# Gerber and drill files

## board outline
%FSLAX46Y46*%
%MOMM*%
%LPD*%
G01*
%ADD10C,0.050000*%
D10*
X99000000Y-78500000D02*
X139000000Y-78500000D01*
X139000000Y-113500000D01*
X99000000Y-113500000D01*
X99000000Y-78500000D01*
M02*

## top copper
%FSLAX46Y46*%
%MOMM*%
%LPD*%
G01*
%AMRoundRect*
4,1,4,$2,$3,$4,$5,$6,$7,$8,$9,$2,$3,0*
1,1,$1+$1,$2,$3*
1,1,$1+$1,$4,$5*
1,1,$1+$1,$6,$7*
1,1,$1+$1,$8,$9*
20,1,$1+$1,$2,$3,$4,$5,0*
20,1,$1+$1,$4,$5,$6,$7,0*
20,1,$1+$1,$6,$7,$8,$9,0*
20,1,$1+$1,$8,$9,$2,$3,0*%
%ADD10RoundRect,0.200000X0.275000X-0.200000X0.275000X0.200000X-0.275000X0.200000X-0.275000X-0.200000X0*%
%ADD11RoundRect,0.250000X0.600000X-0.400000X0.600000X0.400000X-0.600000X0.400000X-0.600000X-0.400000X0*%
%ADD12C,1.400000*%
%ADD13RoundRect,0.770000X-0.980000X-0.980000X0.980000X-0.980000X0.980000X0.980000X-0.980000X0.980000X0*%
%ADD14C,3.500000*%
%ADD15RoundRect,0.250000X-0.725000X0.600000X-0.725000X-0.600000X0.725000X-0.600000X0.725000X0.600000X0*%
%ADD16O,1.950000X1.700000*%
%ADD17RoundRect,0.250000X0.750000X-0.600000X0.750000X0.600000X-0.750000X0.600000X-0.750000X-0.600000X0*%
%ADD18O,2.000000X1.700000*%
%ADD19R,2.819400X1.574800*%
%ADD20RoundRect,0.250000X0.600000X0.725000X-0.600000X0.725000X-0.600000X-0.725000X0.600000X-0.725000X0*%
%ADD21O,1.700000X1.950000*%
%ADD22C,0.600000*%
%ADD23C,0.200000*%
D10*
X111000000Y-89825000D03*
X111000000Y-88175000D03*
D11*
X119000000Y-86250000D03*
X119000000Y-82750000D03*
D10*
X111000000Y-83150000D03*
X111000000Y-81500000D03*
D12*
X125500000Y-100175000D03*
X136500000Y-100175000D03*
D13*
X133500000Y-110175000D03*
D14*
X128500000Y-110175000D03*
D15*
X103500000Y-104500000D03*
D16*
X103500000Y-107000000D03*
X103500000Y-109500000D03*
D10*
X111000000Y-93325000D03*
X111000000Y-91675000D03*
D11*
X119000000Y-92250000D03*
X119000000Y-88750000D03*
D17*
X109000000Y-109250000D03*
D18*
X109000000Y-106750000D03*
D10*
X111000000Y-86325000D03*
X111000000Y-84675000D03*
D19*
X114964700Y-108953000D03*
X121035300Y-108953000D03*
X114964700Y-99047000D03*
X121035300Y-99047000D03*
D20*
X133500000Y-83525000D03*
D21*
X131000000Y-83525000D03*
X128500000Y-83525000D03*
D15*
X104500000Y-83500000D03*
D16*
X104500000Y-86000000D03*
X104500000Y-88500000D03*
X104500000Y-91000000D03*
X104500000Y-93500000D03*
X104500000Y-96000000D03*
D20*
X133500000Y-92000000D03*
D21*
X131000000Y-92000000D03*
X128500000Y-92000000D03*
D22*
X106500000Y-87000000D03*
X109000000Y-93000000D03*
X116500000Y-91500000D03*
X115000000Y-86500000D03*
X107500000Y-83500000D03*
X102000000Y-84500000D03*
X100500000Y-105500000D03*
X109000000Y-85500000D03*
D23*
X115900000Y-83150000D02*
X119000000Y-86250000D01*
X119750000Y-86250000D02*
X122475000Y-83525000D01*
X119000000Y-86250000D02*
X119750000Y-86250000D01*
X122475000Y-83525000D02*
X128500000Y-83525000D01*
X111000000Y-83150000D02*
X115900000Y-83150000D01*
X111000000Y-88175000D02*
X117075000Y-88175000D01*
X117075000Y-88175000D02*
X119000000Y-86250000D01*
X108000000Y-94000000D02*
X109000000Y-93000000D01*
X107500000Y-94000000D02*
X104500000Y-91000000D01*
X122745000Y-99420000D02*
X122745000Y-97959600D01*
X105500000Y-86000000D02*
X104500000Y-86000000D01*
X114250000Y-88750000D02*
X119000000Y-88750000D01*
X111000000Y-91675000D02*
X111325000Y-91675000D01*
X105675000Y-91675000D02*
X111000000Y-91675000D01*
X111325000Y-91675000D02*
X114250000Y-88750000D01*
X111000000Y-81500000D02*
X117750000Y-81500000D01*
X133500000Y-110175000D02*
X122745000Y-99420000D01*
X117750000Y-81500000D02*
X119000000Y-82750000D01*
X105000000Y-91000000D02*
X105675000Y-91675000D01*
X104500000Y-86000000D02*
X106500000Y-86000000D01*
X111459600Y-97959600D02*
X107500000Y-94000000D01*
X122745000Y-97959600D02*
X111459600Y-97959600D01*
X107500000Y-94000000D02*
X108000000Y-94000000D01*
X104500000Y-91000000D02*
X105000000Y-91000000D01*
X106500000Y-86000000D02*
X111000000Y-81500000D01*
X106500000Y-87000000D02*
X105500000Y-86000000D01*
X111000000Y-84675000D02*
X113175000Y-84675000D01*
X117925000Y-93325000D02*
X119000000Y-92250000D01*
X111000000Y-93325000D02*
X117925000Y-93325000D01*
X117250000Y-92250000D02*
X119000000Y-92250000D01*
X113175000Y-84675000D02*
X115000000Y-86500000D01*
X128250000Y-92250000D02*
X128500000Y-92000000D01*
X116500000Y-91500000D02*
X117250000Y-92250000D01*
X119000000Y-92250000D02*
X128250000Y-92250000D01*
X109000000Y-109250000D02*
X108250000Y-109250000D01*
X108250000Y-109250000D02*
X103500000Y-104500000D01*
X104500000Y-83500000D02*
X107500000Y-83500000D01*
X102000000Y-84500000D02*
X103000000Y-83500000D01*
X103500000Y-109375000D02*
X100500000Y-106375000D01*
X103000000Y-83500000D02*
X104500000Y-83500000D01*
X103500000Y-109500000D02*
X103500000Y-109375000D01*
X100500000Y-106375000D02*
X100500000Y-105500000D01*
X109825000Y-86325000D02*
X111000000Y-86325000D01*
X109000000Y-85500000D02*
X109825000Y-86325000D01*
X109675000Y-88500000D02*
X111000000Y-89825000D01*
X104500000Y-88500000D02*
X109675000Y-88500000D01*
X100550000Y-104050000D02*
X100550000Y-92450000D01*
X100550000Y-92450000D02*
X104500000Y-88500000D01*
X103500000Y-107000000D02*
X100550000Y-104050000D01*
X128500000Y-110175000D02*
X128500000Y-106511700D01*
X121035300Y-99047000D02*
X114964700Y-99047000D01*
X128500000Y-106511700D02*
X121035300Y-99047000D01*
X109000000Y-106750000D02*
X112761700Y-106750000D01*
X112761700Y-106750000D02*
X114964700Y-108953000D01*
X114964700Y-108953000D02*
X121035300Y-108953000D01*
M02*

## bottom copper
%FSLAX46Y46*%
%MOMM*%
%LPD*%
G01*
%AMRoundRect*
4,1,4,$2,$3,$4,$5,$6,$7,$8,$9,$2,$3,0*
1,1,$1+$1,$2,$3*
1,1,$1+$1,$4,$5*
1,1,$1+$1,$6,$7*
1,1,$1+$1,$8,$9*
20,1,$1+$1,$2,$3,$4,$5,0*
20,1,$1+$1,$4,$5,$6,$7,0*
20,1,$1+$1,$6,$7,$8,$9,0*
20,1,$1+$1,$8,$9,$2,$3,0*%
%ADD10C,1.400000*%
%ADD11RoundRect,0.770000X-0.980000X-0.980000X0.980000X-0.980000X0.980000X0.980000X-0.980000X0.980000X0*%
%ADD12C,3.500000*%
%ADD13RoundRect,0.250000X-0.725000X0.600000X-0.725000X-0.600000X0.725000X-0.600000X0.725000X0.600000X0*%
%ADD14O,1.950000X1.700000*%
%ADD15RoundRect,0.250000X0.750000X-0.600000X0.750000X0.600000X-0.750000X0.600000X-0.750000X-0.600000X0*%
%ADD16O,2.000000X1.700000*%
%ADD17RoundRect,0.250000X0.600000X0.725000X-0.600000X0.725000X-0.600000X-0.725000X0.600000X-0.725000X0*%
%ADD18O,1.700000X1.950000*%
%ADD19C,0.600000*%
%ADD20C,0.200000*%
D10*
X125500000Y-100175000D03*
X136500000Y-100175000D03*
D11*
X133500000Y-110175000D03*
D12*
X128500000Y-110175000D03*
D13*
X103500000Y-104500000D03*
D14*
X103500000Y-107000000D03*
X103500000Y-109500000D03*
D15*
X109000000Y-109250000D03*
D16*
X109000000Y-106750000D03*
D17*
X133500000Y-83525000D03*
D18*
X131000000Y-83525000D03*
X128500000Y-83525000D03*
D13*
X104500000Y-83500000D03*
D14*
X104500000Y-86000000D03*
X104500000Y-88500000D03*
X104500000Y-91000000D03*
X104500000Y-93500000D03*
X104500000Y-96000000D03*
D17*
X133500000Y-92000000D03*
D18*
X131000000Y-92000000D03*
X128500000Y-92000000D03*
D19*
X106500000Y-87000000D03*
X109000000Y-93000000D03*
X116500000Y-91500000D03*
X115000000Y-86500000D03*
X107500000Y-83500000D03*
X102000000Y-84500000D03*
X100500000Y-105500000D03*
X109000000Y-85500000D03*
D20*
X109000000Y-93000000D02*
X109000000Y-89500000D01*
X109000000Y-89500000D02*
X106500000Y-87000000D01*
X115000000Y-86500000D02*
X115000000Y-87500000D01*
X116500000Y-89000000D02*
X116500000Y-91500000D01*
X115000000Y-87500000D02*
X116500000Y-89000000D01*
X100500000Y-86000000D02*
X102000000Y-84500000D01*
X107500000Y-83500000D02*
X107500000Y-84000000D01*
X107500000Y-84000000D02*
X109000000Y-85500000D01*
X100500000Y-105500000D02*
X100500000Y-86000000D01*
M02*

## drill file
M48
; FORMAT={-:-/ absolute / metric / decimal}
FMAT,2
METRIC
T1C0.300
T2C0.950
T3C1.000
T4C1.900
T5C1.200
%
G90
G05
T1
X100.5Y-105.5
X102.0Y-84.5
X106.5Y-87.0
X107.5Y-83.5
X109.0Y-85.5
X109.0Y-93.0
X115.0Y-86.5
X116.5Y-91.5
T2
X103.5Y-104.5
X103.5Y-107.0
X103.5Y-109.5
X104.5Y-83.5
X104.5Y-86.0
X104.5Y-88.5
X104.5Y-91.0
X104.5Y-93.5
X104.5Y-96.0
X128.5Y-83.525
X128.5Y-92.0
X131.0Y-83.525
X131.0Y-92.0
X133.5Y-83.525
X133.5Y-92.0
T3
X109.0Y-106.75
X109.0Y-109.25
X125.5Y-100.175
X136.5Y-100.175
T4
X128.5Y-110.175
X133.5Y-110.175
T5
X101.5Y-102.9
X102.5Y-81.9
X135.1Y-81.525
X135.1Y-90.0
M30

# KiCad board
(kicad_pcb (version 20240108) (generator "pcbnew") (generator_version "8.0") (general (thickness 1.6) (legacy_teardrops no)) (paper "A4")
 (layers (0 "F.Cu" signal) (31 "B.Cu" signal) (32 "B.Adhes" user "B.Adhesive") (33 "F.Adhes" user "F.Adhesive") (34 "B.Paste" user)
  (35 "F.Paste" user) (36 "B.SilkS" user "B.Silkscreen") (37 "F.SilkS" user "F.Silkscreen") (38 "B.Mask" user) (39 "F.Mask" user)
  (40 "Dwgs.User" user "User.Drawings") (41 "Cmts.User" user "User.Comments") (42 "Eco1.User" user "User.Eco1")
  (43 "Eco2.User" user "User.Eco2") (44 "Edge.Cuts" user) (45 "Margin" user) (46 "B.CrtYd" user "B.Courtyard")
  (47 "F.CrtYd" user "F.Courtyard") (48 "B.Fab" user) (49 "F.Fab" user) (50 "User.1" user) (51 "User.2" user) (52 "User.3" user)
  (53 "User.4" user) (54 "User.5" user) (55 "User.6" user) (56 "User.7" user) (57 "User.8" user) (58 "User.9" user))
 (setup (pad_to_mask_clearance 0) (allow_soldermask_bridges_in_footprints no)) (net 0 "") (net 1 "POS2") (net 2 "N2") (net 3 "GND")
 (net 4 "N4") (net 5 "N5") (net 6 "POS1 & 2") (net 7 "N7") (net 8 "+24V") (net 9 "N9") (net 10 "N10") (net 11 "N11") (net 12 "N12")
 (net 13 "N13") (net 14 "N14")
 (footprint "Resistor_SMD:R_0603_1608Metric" (layer "F.Cu") (at 111 89 90)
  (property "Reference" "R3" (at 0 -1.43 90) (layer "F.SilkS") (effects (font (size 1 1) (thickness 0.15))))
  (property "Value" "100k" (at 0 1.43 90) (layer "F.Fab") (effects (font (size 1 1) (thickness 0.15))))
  (pad "1" smd roundrect (at -0.825 0 90) (size 0.8 0.95) (layers "F.Cu" "F.Paste" "F.Mask") (roundrect_rratio 0.25) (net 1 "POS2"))
  (pad "2" smd roundrect (at 0.825 0 90) (size 0.8 0.95) (layers "F.Cu" "F.Paste" "F.Mask") (roundrect_rratio 0.25) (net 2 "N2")))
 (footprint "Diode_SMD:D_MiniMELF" (layer "F.Cu") (at 119 84.5 90)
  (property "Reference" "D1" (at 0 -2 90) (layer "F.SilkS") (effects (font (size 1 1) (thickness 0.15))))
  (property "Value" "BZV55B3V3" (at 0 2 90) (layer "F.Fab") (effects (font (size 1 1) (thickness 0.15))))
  (pad "1" smd roundrect (at -1.75 0 90) (size 1.3 1.7) (layers "F.Cu" "F.Paste" "F.Mask") (roundrect_rratio 0.1923076923) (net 2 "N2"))
  (pad "2" smd roundrect (at 1.75 0 90) (size 1.3 1.7) (layers "F.Cu" "F.Paste" "F.Mask") (roundrect_rratio 0.1923076923) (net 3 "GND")))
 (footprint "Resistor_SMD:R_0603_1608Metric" (layer "F.Cu") (at 111 82.325 90)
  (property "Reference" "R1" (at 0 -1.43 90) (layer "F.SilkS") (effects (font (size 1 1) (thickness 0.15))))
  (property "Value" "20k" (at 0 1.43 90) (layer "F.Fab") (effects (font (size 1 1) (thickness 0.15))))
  (pad "1" smd roundrect (at -0.825 0 90) (size 0.8 0.95) (layers "F.Cu" "F.Paste" "F.Mask") (roundrect_rratio 0.25) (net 2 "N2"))
  (pad "2" smd roundrect (at 0.825 0 90) (size 0.8 0.95) (layers "F.Cu" "F.Paste" "F.Mask") (roundrect_rratio 0.25) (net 3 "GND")))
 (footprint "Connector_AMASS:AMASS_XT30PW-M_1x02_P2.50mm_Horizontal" (layer "F.Cu") (at 133.5 110.175)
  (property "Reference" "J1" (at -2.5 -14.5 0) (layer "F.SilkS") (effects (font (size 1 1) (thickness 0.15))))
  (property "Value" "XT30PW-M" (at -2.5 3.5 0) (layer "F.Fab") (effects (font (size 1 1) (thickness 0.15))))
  (pad "" thru_hole circle (at -8 -10) (size 1.4 1.4) (drill 1) (layers "*.Cu" "*.Mask") (remove_unused_layers no))
  (pad "" thru_hole circle (at 3 -10) (size 1.4 1.4) (drill 1) (layers "*.Cu" "*.Mask") (remove_unused_layers no))
  (pad "1" thru_hole roundrect (at 0 0) (size 3.5 3.5) (drill 1.9) (layers "*.Cu" "*.Mask") (remove_unused_layers no)
   (roundrect_rratio 0.22) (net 3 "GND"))
  (pad "2" thru_hole circle (at -5 0) (size 3.5 3.5) (drill 1.9) (layers "*.Cu" "*.Mask") (remove_unused_layers no) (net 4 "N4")))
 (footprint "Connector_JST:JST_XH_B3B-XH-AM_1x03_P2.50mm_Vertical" (layer "F.Cu") (at 103.5 104.5 -90)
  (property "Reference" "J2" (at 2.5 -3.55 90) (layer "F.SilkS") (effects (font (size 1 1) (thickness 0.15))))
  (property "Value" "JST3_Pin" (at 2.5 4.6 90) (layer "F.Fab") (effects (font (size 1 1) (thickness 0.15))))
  (pad "" np_thru_hole circle (at -1.6 2 270) (size 1.2 1.2) (drill 1.2) (layers "*.Cu" "*.Mask"))
  (pad "1" thru_hole roundrect (at 0 0 270) (size 1.7 1.95) (drill 0.95) (layers "*.Cu" "*.Mask") (remove_unused_layers no)
   (roundrect_rratio 0.147059) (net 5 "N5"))
  (pad "2" thru_hole oval (at 2.5 0 270) (size 1.7 1.95) (drill 0.95) (layers "*.Cu" "*.Mask") (remove_unused_layers no) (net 1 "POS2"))
  (pad "3" thru_hole oval (at 5 0 270) (size 1.7 1.95) (drill 0.95) (layers "*.Cu" "*.Mask") (remove_unused_layers no) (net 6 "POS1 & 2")))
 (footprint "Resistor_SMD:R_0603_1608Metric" (layer "F.Cu") (at 111 92.5 90)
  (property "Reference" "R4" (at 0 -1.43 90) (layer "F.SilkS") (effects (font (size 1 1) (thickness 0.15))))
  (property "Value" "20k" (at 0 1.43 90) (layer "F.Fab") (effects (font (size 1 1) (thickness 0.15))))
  (pad "1" smd roundrect (at -0.825 0 90) (size 0.8 0.95) (layers "F.Cu" "F.Paste" "F.Mask") (roundrect_rratio 0.25) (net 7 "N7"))
  (pad "2" smd roundrect (at 0.825 0 90) (size 0.8 0.95) (layers "F.Cu" "F.Paste" "F.Mask") (roundrect_rratio 0.25) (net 3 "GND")))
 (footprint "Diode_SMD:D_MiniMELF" (layer "F.Cu") (at 119 90.5 90)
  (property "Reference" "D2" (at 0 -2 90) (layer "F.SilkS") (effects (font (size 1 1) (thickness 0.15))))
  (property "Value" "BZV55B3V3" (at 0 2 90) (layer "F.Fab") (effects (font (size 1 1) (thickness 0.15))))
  (pad "1" smd roundrect (at -1.75 0 90) (size 1.3 1.7) (layers "F.Cu" "F.Paste" "F.Mask") (roundrect_rratio 0.1923076923) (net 7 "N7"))
  (pad "2" smd roundrect (at 1.75 0 90) (size 1.3 1.7) (layers "F.Cu" "F.Paste" "F.Mask") (roundrect_rratio 0.1923076923) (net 3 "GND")))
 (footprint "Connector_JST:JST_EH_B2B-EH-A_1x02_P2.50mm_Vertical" (layer "F.Cu") (at 109 109.25 90)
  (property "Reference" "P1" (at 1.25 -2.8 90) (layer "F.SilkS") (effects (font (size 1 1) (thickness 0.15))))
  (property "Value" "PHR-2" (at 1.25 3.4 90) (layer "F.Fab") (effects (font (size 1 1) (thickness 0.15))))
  (pad "1" thru_hole roundrect (at 0 0 90) (size 1.7 2) (drill 1) (layers "*.Cu" "*.Mask") (remove_unused_layers no)
   (roundrect_rratio 0.147059) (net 5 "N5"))
  (pad "2" thru_hole oval (at 2.5 0 90) (size 1.7 2) (drill 1) (layers "*.Cu" "*.Mask") (remove_unused_layers no) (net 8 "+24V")))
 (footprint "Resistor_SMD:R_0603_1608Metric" (layer "F.Cu") (at 111 85.5 90)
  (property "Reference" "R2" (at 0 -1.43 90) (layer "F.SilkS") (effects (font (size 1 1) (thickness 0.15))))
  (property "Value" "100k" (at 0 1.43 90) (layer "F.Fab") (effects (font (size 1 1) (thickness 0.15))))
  (pad "1" smd roundrect (at -0.825 0 90) (size 0.8 0.95) (layers "F.Cu" "F.Paste" "F.Mask") (roundrect_rratio 0.25) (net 6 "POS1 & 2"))
  (pad "2" smd roundrect (at 0.825 0 90) (size 0.8 0.95) (layers "F.Cu" "F.Paste" "F.Mask") (roundrect_rratio 0.25) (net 7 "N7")))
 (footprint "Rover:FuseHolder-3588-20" (layer "F.Cu") (at 118 104 90)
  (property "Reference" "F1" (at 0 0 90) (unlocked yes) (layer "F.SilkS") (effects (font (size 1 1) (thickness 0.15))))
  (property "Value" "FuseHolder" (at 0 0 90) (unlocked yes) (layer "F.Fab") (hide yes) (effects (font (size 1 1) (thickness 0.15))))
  (pad "1" smd rect (at -4.953 -3.0353 90) (size 1.5748 2.8194) (layers "F.Cu" "F.Paste" "F.Mask") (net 8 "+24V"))
  (pad "1" smd rect (at -4.953 3.0353 90) (size 1.5748 2.8194) (layers "F.Cu" "F.Paste" "F.Mask") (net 8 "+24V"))
  (pad "2" smd rect (at 4.953 -3.0353 90) (size 1.5748 2.8194) (layers "F.Cu" "F.Paste" "F.Mask") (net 4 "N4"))
  (pad "2" smd rect (at 4.953 3.0353 90) (size 1.5748 2.8194) (layers "F.Cu" "F.Paste" "F.Mask") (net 4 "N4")))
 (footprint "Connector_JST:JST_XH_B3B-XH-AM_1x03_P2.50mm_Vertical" (layer "F.Cu") (at 133.5 83.525 180)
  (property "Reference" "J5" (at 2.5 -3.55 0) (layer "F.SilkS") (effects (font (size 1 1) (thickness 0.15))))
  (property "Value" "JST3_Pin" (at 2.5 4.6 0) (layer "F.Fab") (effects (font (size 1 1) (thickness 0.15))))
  (pad "" np_thru_hole circle (at -1.6 2 180) (size 1.2 1.2) (drill 1.2) (layers "*.Cu" "*.Mask"))
  (pad "1" thru_hole roundrect (at 0 0 180) (size 1.7 1.95) (drill 0.95) (layers "*.Cu" "*.Mask") (remove_unused_layers no)
   (roundrect_rratio 0.147059) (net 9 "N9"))
  (pad "2" thru_hole oval (at 2.5 0 180) (size 1.7 1.95) (drill 0.95) (layers "*.Cu" "*.Mask") (remove_unused_layers no) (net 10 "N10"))
  (pad "3" thru_hole oval (at 5 0 180) (size 1.7 1.95) (drill 0.95) (layers "*.Cu" "*.Mask") (remove_unused_layers no) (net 2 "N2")))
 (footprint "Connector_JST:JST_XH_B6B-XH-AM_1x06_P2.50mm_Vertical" (layer "F.Cu") (at 104.5 83.5 -90)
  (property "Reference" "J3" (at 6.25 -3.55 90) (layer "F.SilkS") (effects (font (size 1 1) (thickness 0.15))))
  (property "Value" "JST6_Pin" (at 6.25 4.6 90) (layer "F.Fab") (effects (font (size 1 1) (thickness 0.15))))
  (pad "" np_thru_hole circle (at -1.6 2 270) (size 1.2 1.2) (drill 1.2) (layers "*.Cu" "*.Mask"))
  (pad "1" thru_hole roundrect (at 0 0 270) (size 1.7 1.95) (drill 0.95) (layers "*.Cu" "*.Mask") (remove_unused_layers no)
   (roundrect_rratio 0.147059) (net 6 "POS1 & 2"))
  (pad "2" thru_hole oval (at 2.5 0 270) (size 1.7 1.95) (drill 0.95) (layers "*.Cu" "*.Mask") (remove_unused_layers no) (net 3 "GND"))
  (pad "3" thru_hole oval (at 5 0 270) (size 1.7 1.95) (drill 0.95) (layers "*.Cu" "*.Mask") (remove_unused_layers no) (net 1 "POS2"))
  (pad "4" thru_hole oval (at 7.5 0 270) (size 1.7 1.95) (drill 0.95) (layers "*.Cu" "*.Mask") (remove_unused_layers no) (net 3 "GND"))
  (pad "5" thru_hole oval (at 10 0 270) (size 1.7 1.95) (drill 0.95) (layers "*.Cu" "*.Mask") (remove_unused_layers no) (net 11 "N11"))
  (pad "6" thru_hole oval (at 12.5 0 270) (size 1.7 1.95) (drill 0.95) (layers "*.Cu" "*.Mask") (remove_unused_layers no) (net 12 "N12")))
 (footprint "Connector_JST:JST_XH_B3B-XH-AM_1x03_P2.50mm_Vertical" (layer "F.Cu") (at 133.5 92 180)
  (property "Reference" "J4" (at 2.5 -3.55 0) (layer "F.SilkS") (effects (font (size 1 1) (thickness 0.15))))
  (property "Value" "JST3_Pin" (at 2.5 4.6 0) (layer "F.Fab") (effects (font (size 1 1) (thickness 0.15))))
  (pad "" np_thru_hole circle (at -1.6 2 180) (size 1.2 1.2) (drill 1.2) (layers "*.Cu" "*.Mask"))
  (pad "1" thru_hole roundrect (at 0 0 180) (size 1.7 1.95) (drill 0.95) (layers "*.Cu" "*.Mask") (remove_unused_layers no)
   (roundrect_rratio 0.147059) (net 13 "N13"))
  (pad "2" thru_hole oval (at 2.5 0 180) (size 1.7 1.95) (drill 0.95) (layers "*.Cu" "*.Mask") (remove_unused_layers no) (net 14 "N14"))
  (pad "3" thru_hole oval (at 5 0 180) (size 1.7 1.95) (drill 0.95) (layers "*.Cu" "*.Mask") (remove_unused_layers no) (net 7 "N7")))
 (gr_rect (start 99 78.5) (end 139 113.5) (stroke (width 0.05) (type default)) (fill none) (layer "Edge.Cuts"))
 (segment (start 115.9 83.15) (end 119 86.25) (width 0.2) (layer "F.Cu") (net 2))
 (segment (start 119.75 86.25) (end 122.475 83.525) (width 0.2) (layer "F.Cu") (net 2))
 (segment (start 119 86.25) (end 119.75 86.25) (width 0.2) (layer "F.Cu") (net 2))
 (segment (start 122.475 83.525) (end 128.5 83.525) (width 0.2) (layer "F.Cu") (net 2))
 (segment (start 111 83.15) (end 115.9 83.15) (width 0.2) (layer "F.Cu") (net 2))
 (segment (start 111 88.175) (end 117.075 88.175) (width 0.2) (layer "F.Cu") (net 2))
 (segment (start 117.075 88.175) (end 119 86.25) (width 0.2) (layer "F.Cu") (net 2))
 (segment (start 108 94) (end 109 93) (width 0.2) (layer "F.Cu") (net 3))
 (segment (start 107.5 94) (end 104.5 91) (width 0.2) (layer "F.Cu") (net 3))
 (segment (start 122.745 99.42) (end 122.745 97.9596) (width 0.2) (layer "F.Cu") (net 3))
 (segment (start 105.5 86) (end 104.5 86) (width 0.2) (layer "F.Cu") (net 3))
 (segment (start 114.25 88.75) (end 119 88.75) (width 0.2) (layer "F.Cu") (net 3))
 (segment (start 111 91.675) (end 111.325 91.675) (width 0.2) (layer "F.Cu") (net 3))
 (segment (start 105.675 91.675) (end 111 91.675) (width 0.2) (layer "F.Cu") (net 3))
 (segment (start 111.325 91.675) (end 114.25 88.75) (width 0.2) (layer "F.Cu") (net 3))
 (segment (start 111 81.5) (end 117.75 81.5) (width 0.2) (layer "F.Cu") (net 3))
 (segment (start 133.5 110.175) (end 122.745 99.42) (width 0.2) (layer "F.Cu") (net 3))
 (segment (start 117.75 81.5) (end 119 82.75) (width 0.2) (layer "F.Cu") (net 3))
 (segment (start 105 91) (end 105.675 91.675) (width 0.2) (layer "F.Cu") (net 3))
 (segment (start 104.5 86) (end 106.5 86) (width 0.2) (layer "F.Cu") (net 3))
 (segment (start 111.4596 97.9596) (end 107.5 94) (width 0.2) (layer "F.Cu") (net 3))
 (segment (start 122.745 97.9596) (end 111.4596 97.9596) (width 0.2) (layer "F.Cu") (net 3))
 (segment (start 107.5 94) (end 108 94) (width 0.2) (layer "F.Cu") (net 3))
 (segment (start 104.5 91) (end 105 91) (width 0.2) (layer "F.Cu") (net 3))
 (segment (start 106.5 86) (end 111 81.5) (width 0.2) (layer "F.Cu") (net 3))
 (segment (start 106.5 87) (end 105.5 86) (width 0.2) (layer "F.Cu") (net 3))
 (via (at 106.5 87) (size 0.6) (drill 0.3) (layers "F.Cu" "B.Cu") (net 3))
 (via (at 109 93) (size 0.6) (drill 0.3) (layers "F.Cu" "B.Cu") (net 3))
 (segment (start 109 93) (end 109 89.5) (width 0.2) (layer "B.Cu") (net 3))
 (segment (start 109 89.5) (end 106.5 87) (width 0.2) (layer "B.Cu") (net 3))
 (segment (start 111 84.675) (end 113.175 84.675) (width 0.2) (layer "F.Cu") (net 7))
 (segment (start 117.925 93.325) (end 119 92.25) (width 0.2) (layer "F.Cu") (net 7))
 (segment (start 111 93.325) (end 117.925 93.325) (width 0.2) (layer "F.Cu") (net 7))
 (segment (start 117.25 92.25) (end 119 92.25) (width 0.2) (layer "F.Cu") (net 7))
 (segment (start 113.175 84.675) (end 115 86.5) (width 0.2) (layer "F.Cu") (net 7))
 (segment (start 128.25 92.25) (end 128.5 92) (width 0.2) (layer "F.Cu") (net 7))
 (segment (start 116.5 91.5) (end 117.25 92.25) (width 0.2) (layer "F.Cu") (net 7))
 (segment (start 119 92.25) (end 128.25 92.25) (width 0.2) (layer "F.Cu") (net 7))
 (via (at 116.5 91.5) (size 0.6) (drill 0.3) (layers "F.Cu" "B.Cu") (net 7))
 (via (at 115 86.5) (size 0.6) (drill 0.3) (layers "F.Cu" "B.Cu") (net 7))
 (segment (start 115 86.5) (end 115 87.5) (width 0.2) (layer "B.Cu") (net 7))
 (segment (start 116.5 89) (end 116.5 91.5) (width 0.2) (layer "B.Cu") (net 7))
 (segment (start 115 87.5) (end 116.5 89) (width 0.2) (layer "B.Cu") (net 7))
 (segment (start 109 109.25) (end 108.25 109.25) (width 0.2) (layer "F.Cu") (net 5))
 (segment (start 108.25 109.25) (end 103.5 104.5) (width 0.2) (layer "F.Cu") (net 5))
 (segment (start 104.5 83.5) (end 107.5 83.5) (width 0.2) (layer "F.Cu") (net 6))
 (segment (start 102 84.5) (end 103 83.5) (width 0.2) (layer "F.Cu") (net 6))
 (segment (start 103.5 109.375) (end 100.5 106.375) (width 0.2) (layer "F.Cu") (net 6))
 (segment (start 103 83.5) (end 104.5 83.5) (width 0.2) (layer "F.Cu") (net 6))
 (segment (start 103.5 109.5) (end 103.5 109.375) (width 0.2) (layer "F.Cu") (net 6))
 (segment (start 100.5 106.375) (end 100.5 105.5) (width 0.2) (layer "F.Cu") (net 6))
 (segment (start 109.825 86.325) (end 111 86.325) (width 0.2) (layer "F.Cu") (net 6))
 (segment (start 109 85.5) (end 109.825 86.325) (width 0.2) (layer "F.Cu") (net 6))
 (via (at 107.5 83.5) (size 0.6) (drill 0.3) (layers "F.Cu" "B.Cu") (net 6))
 (via (at 102 84.5) (size 0.6) (drill 0.3) (layers "F.Cu" "B.Cu") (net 6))
 (via (at 100.5 105.5) (size 0.6) (drill 0.3) (layers "F.Cu" "B.Cu") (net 6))
 (via (at 109 85.5) (size 0.6) (drill 0.3) (layers "F.Cu" "B.Cu") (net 6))
 (segment (start 100.5 86) (end 102 84.5) (width 0.2) (layer "B.Cu") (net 6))
 (segment (start 107.5 83.5) (end 107.5 84) (width 0.2) (layer "B.Cu") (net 6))
 (segment (start 107.5 84) (end 109 85.5) (width 0.2) (layer "B.Cu") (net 6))
 (segment (start 100.5 105.5) (end 100.5 86) (width 0.2) (layer "B.Cu") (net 6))
 (segment (start 109.675 88.5) (end 111 89.825) (width 0.2) (layer "F.Cu") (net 1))
 (segment (start 104.5 88.5) (end 109.675 88.5) (width 0.2) (layer "F.Cu") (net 1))
 (segment (start 100.55 104.05) (end 100.55 92.45) (width 0.2) (layer "F.Cu") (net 1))
 (segment (start 100.55 92.45) (end 104.5 88.5) (width 0.2) (layer "F.Cu") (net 1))
 (segment (start 103.5 107) (end 100.55 104.05) (width 0.2) (layer "F.Cu") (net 1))
 (segment (start 128.5 110.175) (end 128.5 106.5117) (width 0.2) (layer "F.Cu") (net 4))
 (segment (start 121.0353 99.047) (end 114.9647 99.047) (width 0.2) (layer "F.Cu") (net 4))
 (segment (start 128.5 106.5117) (end 121.0353 99.047) (width 0.2) (layer "F.Cu") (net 4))
 (segment (start 109 106.75) (end 112.7617 106.75) (width 0.2) (layer "F.Cu") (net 8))
 (segment (start 112.7617 106.75) (end 114.9647 108.953) (width 0.2) (layer "F.Cu") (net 8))
 (segment (start 114.9647 108.953) (end 121.0353 108.953) (width 0.2) (layer "F.Cu") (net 8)))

